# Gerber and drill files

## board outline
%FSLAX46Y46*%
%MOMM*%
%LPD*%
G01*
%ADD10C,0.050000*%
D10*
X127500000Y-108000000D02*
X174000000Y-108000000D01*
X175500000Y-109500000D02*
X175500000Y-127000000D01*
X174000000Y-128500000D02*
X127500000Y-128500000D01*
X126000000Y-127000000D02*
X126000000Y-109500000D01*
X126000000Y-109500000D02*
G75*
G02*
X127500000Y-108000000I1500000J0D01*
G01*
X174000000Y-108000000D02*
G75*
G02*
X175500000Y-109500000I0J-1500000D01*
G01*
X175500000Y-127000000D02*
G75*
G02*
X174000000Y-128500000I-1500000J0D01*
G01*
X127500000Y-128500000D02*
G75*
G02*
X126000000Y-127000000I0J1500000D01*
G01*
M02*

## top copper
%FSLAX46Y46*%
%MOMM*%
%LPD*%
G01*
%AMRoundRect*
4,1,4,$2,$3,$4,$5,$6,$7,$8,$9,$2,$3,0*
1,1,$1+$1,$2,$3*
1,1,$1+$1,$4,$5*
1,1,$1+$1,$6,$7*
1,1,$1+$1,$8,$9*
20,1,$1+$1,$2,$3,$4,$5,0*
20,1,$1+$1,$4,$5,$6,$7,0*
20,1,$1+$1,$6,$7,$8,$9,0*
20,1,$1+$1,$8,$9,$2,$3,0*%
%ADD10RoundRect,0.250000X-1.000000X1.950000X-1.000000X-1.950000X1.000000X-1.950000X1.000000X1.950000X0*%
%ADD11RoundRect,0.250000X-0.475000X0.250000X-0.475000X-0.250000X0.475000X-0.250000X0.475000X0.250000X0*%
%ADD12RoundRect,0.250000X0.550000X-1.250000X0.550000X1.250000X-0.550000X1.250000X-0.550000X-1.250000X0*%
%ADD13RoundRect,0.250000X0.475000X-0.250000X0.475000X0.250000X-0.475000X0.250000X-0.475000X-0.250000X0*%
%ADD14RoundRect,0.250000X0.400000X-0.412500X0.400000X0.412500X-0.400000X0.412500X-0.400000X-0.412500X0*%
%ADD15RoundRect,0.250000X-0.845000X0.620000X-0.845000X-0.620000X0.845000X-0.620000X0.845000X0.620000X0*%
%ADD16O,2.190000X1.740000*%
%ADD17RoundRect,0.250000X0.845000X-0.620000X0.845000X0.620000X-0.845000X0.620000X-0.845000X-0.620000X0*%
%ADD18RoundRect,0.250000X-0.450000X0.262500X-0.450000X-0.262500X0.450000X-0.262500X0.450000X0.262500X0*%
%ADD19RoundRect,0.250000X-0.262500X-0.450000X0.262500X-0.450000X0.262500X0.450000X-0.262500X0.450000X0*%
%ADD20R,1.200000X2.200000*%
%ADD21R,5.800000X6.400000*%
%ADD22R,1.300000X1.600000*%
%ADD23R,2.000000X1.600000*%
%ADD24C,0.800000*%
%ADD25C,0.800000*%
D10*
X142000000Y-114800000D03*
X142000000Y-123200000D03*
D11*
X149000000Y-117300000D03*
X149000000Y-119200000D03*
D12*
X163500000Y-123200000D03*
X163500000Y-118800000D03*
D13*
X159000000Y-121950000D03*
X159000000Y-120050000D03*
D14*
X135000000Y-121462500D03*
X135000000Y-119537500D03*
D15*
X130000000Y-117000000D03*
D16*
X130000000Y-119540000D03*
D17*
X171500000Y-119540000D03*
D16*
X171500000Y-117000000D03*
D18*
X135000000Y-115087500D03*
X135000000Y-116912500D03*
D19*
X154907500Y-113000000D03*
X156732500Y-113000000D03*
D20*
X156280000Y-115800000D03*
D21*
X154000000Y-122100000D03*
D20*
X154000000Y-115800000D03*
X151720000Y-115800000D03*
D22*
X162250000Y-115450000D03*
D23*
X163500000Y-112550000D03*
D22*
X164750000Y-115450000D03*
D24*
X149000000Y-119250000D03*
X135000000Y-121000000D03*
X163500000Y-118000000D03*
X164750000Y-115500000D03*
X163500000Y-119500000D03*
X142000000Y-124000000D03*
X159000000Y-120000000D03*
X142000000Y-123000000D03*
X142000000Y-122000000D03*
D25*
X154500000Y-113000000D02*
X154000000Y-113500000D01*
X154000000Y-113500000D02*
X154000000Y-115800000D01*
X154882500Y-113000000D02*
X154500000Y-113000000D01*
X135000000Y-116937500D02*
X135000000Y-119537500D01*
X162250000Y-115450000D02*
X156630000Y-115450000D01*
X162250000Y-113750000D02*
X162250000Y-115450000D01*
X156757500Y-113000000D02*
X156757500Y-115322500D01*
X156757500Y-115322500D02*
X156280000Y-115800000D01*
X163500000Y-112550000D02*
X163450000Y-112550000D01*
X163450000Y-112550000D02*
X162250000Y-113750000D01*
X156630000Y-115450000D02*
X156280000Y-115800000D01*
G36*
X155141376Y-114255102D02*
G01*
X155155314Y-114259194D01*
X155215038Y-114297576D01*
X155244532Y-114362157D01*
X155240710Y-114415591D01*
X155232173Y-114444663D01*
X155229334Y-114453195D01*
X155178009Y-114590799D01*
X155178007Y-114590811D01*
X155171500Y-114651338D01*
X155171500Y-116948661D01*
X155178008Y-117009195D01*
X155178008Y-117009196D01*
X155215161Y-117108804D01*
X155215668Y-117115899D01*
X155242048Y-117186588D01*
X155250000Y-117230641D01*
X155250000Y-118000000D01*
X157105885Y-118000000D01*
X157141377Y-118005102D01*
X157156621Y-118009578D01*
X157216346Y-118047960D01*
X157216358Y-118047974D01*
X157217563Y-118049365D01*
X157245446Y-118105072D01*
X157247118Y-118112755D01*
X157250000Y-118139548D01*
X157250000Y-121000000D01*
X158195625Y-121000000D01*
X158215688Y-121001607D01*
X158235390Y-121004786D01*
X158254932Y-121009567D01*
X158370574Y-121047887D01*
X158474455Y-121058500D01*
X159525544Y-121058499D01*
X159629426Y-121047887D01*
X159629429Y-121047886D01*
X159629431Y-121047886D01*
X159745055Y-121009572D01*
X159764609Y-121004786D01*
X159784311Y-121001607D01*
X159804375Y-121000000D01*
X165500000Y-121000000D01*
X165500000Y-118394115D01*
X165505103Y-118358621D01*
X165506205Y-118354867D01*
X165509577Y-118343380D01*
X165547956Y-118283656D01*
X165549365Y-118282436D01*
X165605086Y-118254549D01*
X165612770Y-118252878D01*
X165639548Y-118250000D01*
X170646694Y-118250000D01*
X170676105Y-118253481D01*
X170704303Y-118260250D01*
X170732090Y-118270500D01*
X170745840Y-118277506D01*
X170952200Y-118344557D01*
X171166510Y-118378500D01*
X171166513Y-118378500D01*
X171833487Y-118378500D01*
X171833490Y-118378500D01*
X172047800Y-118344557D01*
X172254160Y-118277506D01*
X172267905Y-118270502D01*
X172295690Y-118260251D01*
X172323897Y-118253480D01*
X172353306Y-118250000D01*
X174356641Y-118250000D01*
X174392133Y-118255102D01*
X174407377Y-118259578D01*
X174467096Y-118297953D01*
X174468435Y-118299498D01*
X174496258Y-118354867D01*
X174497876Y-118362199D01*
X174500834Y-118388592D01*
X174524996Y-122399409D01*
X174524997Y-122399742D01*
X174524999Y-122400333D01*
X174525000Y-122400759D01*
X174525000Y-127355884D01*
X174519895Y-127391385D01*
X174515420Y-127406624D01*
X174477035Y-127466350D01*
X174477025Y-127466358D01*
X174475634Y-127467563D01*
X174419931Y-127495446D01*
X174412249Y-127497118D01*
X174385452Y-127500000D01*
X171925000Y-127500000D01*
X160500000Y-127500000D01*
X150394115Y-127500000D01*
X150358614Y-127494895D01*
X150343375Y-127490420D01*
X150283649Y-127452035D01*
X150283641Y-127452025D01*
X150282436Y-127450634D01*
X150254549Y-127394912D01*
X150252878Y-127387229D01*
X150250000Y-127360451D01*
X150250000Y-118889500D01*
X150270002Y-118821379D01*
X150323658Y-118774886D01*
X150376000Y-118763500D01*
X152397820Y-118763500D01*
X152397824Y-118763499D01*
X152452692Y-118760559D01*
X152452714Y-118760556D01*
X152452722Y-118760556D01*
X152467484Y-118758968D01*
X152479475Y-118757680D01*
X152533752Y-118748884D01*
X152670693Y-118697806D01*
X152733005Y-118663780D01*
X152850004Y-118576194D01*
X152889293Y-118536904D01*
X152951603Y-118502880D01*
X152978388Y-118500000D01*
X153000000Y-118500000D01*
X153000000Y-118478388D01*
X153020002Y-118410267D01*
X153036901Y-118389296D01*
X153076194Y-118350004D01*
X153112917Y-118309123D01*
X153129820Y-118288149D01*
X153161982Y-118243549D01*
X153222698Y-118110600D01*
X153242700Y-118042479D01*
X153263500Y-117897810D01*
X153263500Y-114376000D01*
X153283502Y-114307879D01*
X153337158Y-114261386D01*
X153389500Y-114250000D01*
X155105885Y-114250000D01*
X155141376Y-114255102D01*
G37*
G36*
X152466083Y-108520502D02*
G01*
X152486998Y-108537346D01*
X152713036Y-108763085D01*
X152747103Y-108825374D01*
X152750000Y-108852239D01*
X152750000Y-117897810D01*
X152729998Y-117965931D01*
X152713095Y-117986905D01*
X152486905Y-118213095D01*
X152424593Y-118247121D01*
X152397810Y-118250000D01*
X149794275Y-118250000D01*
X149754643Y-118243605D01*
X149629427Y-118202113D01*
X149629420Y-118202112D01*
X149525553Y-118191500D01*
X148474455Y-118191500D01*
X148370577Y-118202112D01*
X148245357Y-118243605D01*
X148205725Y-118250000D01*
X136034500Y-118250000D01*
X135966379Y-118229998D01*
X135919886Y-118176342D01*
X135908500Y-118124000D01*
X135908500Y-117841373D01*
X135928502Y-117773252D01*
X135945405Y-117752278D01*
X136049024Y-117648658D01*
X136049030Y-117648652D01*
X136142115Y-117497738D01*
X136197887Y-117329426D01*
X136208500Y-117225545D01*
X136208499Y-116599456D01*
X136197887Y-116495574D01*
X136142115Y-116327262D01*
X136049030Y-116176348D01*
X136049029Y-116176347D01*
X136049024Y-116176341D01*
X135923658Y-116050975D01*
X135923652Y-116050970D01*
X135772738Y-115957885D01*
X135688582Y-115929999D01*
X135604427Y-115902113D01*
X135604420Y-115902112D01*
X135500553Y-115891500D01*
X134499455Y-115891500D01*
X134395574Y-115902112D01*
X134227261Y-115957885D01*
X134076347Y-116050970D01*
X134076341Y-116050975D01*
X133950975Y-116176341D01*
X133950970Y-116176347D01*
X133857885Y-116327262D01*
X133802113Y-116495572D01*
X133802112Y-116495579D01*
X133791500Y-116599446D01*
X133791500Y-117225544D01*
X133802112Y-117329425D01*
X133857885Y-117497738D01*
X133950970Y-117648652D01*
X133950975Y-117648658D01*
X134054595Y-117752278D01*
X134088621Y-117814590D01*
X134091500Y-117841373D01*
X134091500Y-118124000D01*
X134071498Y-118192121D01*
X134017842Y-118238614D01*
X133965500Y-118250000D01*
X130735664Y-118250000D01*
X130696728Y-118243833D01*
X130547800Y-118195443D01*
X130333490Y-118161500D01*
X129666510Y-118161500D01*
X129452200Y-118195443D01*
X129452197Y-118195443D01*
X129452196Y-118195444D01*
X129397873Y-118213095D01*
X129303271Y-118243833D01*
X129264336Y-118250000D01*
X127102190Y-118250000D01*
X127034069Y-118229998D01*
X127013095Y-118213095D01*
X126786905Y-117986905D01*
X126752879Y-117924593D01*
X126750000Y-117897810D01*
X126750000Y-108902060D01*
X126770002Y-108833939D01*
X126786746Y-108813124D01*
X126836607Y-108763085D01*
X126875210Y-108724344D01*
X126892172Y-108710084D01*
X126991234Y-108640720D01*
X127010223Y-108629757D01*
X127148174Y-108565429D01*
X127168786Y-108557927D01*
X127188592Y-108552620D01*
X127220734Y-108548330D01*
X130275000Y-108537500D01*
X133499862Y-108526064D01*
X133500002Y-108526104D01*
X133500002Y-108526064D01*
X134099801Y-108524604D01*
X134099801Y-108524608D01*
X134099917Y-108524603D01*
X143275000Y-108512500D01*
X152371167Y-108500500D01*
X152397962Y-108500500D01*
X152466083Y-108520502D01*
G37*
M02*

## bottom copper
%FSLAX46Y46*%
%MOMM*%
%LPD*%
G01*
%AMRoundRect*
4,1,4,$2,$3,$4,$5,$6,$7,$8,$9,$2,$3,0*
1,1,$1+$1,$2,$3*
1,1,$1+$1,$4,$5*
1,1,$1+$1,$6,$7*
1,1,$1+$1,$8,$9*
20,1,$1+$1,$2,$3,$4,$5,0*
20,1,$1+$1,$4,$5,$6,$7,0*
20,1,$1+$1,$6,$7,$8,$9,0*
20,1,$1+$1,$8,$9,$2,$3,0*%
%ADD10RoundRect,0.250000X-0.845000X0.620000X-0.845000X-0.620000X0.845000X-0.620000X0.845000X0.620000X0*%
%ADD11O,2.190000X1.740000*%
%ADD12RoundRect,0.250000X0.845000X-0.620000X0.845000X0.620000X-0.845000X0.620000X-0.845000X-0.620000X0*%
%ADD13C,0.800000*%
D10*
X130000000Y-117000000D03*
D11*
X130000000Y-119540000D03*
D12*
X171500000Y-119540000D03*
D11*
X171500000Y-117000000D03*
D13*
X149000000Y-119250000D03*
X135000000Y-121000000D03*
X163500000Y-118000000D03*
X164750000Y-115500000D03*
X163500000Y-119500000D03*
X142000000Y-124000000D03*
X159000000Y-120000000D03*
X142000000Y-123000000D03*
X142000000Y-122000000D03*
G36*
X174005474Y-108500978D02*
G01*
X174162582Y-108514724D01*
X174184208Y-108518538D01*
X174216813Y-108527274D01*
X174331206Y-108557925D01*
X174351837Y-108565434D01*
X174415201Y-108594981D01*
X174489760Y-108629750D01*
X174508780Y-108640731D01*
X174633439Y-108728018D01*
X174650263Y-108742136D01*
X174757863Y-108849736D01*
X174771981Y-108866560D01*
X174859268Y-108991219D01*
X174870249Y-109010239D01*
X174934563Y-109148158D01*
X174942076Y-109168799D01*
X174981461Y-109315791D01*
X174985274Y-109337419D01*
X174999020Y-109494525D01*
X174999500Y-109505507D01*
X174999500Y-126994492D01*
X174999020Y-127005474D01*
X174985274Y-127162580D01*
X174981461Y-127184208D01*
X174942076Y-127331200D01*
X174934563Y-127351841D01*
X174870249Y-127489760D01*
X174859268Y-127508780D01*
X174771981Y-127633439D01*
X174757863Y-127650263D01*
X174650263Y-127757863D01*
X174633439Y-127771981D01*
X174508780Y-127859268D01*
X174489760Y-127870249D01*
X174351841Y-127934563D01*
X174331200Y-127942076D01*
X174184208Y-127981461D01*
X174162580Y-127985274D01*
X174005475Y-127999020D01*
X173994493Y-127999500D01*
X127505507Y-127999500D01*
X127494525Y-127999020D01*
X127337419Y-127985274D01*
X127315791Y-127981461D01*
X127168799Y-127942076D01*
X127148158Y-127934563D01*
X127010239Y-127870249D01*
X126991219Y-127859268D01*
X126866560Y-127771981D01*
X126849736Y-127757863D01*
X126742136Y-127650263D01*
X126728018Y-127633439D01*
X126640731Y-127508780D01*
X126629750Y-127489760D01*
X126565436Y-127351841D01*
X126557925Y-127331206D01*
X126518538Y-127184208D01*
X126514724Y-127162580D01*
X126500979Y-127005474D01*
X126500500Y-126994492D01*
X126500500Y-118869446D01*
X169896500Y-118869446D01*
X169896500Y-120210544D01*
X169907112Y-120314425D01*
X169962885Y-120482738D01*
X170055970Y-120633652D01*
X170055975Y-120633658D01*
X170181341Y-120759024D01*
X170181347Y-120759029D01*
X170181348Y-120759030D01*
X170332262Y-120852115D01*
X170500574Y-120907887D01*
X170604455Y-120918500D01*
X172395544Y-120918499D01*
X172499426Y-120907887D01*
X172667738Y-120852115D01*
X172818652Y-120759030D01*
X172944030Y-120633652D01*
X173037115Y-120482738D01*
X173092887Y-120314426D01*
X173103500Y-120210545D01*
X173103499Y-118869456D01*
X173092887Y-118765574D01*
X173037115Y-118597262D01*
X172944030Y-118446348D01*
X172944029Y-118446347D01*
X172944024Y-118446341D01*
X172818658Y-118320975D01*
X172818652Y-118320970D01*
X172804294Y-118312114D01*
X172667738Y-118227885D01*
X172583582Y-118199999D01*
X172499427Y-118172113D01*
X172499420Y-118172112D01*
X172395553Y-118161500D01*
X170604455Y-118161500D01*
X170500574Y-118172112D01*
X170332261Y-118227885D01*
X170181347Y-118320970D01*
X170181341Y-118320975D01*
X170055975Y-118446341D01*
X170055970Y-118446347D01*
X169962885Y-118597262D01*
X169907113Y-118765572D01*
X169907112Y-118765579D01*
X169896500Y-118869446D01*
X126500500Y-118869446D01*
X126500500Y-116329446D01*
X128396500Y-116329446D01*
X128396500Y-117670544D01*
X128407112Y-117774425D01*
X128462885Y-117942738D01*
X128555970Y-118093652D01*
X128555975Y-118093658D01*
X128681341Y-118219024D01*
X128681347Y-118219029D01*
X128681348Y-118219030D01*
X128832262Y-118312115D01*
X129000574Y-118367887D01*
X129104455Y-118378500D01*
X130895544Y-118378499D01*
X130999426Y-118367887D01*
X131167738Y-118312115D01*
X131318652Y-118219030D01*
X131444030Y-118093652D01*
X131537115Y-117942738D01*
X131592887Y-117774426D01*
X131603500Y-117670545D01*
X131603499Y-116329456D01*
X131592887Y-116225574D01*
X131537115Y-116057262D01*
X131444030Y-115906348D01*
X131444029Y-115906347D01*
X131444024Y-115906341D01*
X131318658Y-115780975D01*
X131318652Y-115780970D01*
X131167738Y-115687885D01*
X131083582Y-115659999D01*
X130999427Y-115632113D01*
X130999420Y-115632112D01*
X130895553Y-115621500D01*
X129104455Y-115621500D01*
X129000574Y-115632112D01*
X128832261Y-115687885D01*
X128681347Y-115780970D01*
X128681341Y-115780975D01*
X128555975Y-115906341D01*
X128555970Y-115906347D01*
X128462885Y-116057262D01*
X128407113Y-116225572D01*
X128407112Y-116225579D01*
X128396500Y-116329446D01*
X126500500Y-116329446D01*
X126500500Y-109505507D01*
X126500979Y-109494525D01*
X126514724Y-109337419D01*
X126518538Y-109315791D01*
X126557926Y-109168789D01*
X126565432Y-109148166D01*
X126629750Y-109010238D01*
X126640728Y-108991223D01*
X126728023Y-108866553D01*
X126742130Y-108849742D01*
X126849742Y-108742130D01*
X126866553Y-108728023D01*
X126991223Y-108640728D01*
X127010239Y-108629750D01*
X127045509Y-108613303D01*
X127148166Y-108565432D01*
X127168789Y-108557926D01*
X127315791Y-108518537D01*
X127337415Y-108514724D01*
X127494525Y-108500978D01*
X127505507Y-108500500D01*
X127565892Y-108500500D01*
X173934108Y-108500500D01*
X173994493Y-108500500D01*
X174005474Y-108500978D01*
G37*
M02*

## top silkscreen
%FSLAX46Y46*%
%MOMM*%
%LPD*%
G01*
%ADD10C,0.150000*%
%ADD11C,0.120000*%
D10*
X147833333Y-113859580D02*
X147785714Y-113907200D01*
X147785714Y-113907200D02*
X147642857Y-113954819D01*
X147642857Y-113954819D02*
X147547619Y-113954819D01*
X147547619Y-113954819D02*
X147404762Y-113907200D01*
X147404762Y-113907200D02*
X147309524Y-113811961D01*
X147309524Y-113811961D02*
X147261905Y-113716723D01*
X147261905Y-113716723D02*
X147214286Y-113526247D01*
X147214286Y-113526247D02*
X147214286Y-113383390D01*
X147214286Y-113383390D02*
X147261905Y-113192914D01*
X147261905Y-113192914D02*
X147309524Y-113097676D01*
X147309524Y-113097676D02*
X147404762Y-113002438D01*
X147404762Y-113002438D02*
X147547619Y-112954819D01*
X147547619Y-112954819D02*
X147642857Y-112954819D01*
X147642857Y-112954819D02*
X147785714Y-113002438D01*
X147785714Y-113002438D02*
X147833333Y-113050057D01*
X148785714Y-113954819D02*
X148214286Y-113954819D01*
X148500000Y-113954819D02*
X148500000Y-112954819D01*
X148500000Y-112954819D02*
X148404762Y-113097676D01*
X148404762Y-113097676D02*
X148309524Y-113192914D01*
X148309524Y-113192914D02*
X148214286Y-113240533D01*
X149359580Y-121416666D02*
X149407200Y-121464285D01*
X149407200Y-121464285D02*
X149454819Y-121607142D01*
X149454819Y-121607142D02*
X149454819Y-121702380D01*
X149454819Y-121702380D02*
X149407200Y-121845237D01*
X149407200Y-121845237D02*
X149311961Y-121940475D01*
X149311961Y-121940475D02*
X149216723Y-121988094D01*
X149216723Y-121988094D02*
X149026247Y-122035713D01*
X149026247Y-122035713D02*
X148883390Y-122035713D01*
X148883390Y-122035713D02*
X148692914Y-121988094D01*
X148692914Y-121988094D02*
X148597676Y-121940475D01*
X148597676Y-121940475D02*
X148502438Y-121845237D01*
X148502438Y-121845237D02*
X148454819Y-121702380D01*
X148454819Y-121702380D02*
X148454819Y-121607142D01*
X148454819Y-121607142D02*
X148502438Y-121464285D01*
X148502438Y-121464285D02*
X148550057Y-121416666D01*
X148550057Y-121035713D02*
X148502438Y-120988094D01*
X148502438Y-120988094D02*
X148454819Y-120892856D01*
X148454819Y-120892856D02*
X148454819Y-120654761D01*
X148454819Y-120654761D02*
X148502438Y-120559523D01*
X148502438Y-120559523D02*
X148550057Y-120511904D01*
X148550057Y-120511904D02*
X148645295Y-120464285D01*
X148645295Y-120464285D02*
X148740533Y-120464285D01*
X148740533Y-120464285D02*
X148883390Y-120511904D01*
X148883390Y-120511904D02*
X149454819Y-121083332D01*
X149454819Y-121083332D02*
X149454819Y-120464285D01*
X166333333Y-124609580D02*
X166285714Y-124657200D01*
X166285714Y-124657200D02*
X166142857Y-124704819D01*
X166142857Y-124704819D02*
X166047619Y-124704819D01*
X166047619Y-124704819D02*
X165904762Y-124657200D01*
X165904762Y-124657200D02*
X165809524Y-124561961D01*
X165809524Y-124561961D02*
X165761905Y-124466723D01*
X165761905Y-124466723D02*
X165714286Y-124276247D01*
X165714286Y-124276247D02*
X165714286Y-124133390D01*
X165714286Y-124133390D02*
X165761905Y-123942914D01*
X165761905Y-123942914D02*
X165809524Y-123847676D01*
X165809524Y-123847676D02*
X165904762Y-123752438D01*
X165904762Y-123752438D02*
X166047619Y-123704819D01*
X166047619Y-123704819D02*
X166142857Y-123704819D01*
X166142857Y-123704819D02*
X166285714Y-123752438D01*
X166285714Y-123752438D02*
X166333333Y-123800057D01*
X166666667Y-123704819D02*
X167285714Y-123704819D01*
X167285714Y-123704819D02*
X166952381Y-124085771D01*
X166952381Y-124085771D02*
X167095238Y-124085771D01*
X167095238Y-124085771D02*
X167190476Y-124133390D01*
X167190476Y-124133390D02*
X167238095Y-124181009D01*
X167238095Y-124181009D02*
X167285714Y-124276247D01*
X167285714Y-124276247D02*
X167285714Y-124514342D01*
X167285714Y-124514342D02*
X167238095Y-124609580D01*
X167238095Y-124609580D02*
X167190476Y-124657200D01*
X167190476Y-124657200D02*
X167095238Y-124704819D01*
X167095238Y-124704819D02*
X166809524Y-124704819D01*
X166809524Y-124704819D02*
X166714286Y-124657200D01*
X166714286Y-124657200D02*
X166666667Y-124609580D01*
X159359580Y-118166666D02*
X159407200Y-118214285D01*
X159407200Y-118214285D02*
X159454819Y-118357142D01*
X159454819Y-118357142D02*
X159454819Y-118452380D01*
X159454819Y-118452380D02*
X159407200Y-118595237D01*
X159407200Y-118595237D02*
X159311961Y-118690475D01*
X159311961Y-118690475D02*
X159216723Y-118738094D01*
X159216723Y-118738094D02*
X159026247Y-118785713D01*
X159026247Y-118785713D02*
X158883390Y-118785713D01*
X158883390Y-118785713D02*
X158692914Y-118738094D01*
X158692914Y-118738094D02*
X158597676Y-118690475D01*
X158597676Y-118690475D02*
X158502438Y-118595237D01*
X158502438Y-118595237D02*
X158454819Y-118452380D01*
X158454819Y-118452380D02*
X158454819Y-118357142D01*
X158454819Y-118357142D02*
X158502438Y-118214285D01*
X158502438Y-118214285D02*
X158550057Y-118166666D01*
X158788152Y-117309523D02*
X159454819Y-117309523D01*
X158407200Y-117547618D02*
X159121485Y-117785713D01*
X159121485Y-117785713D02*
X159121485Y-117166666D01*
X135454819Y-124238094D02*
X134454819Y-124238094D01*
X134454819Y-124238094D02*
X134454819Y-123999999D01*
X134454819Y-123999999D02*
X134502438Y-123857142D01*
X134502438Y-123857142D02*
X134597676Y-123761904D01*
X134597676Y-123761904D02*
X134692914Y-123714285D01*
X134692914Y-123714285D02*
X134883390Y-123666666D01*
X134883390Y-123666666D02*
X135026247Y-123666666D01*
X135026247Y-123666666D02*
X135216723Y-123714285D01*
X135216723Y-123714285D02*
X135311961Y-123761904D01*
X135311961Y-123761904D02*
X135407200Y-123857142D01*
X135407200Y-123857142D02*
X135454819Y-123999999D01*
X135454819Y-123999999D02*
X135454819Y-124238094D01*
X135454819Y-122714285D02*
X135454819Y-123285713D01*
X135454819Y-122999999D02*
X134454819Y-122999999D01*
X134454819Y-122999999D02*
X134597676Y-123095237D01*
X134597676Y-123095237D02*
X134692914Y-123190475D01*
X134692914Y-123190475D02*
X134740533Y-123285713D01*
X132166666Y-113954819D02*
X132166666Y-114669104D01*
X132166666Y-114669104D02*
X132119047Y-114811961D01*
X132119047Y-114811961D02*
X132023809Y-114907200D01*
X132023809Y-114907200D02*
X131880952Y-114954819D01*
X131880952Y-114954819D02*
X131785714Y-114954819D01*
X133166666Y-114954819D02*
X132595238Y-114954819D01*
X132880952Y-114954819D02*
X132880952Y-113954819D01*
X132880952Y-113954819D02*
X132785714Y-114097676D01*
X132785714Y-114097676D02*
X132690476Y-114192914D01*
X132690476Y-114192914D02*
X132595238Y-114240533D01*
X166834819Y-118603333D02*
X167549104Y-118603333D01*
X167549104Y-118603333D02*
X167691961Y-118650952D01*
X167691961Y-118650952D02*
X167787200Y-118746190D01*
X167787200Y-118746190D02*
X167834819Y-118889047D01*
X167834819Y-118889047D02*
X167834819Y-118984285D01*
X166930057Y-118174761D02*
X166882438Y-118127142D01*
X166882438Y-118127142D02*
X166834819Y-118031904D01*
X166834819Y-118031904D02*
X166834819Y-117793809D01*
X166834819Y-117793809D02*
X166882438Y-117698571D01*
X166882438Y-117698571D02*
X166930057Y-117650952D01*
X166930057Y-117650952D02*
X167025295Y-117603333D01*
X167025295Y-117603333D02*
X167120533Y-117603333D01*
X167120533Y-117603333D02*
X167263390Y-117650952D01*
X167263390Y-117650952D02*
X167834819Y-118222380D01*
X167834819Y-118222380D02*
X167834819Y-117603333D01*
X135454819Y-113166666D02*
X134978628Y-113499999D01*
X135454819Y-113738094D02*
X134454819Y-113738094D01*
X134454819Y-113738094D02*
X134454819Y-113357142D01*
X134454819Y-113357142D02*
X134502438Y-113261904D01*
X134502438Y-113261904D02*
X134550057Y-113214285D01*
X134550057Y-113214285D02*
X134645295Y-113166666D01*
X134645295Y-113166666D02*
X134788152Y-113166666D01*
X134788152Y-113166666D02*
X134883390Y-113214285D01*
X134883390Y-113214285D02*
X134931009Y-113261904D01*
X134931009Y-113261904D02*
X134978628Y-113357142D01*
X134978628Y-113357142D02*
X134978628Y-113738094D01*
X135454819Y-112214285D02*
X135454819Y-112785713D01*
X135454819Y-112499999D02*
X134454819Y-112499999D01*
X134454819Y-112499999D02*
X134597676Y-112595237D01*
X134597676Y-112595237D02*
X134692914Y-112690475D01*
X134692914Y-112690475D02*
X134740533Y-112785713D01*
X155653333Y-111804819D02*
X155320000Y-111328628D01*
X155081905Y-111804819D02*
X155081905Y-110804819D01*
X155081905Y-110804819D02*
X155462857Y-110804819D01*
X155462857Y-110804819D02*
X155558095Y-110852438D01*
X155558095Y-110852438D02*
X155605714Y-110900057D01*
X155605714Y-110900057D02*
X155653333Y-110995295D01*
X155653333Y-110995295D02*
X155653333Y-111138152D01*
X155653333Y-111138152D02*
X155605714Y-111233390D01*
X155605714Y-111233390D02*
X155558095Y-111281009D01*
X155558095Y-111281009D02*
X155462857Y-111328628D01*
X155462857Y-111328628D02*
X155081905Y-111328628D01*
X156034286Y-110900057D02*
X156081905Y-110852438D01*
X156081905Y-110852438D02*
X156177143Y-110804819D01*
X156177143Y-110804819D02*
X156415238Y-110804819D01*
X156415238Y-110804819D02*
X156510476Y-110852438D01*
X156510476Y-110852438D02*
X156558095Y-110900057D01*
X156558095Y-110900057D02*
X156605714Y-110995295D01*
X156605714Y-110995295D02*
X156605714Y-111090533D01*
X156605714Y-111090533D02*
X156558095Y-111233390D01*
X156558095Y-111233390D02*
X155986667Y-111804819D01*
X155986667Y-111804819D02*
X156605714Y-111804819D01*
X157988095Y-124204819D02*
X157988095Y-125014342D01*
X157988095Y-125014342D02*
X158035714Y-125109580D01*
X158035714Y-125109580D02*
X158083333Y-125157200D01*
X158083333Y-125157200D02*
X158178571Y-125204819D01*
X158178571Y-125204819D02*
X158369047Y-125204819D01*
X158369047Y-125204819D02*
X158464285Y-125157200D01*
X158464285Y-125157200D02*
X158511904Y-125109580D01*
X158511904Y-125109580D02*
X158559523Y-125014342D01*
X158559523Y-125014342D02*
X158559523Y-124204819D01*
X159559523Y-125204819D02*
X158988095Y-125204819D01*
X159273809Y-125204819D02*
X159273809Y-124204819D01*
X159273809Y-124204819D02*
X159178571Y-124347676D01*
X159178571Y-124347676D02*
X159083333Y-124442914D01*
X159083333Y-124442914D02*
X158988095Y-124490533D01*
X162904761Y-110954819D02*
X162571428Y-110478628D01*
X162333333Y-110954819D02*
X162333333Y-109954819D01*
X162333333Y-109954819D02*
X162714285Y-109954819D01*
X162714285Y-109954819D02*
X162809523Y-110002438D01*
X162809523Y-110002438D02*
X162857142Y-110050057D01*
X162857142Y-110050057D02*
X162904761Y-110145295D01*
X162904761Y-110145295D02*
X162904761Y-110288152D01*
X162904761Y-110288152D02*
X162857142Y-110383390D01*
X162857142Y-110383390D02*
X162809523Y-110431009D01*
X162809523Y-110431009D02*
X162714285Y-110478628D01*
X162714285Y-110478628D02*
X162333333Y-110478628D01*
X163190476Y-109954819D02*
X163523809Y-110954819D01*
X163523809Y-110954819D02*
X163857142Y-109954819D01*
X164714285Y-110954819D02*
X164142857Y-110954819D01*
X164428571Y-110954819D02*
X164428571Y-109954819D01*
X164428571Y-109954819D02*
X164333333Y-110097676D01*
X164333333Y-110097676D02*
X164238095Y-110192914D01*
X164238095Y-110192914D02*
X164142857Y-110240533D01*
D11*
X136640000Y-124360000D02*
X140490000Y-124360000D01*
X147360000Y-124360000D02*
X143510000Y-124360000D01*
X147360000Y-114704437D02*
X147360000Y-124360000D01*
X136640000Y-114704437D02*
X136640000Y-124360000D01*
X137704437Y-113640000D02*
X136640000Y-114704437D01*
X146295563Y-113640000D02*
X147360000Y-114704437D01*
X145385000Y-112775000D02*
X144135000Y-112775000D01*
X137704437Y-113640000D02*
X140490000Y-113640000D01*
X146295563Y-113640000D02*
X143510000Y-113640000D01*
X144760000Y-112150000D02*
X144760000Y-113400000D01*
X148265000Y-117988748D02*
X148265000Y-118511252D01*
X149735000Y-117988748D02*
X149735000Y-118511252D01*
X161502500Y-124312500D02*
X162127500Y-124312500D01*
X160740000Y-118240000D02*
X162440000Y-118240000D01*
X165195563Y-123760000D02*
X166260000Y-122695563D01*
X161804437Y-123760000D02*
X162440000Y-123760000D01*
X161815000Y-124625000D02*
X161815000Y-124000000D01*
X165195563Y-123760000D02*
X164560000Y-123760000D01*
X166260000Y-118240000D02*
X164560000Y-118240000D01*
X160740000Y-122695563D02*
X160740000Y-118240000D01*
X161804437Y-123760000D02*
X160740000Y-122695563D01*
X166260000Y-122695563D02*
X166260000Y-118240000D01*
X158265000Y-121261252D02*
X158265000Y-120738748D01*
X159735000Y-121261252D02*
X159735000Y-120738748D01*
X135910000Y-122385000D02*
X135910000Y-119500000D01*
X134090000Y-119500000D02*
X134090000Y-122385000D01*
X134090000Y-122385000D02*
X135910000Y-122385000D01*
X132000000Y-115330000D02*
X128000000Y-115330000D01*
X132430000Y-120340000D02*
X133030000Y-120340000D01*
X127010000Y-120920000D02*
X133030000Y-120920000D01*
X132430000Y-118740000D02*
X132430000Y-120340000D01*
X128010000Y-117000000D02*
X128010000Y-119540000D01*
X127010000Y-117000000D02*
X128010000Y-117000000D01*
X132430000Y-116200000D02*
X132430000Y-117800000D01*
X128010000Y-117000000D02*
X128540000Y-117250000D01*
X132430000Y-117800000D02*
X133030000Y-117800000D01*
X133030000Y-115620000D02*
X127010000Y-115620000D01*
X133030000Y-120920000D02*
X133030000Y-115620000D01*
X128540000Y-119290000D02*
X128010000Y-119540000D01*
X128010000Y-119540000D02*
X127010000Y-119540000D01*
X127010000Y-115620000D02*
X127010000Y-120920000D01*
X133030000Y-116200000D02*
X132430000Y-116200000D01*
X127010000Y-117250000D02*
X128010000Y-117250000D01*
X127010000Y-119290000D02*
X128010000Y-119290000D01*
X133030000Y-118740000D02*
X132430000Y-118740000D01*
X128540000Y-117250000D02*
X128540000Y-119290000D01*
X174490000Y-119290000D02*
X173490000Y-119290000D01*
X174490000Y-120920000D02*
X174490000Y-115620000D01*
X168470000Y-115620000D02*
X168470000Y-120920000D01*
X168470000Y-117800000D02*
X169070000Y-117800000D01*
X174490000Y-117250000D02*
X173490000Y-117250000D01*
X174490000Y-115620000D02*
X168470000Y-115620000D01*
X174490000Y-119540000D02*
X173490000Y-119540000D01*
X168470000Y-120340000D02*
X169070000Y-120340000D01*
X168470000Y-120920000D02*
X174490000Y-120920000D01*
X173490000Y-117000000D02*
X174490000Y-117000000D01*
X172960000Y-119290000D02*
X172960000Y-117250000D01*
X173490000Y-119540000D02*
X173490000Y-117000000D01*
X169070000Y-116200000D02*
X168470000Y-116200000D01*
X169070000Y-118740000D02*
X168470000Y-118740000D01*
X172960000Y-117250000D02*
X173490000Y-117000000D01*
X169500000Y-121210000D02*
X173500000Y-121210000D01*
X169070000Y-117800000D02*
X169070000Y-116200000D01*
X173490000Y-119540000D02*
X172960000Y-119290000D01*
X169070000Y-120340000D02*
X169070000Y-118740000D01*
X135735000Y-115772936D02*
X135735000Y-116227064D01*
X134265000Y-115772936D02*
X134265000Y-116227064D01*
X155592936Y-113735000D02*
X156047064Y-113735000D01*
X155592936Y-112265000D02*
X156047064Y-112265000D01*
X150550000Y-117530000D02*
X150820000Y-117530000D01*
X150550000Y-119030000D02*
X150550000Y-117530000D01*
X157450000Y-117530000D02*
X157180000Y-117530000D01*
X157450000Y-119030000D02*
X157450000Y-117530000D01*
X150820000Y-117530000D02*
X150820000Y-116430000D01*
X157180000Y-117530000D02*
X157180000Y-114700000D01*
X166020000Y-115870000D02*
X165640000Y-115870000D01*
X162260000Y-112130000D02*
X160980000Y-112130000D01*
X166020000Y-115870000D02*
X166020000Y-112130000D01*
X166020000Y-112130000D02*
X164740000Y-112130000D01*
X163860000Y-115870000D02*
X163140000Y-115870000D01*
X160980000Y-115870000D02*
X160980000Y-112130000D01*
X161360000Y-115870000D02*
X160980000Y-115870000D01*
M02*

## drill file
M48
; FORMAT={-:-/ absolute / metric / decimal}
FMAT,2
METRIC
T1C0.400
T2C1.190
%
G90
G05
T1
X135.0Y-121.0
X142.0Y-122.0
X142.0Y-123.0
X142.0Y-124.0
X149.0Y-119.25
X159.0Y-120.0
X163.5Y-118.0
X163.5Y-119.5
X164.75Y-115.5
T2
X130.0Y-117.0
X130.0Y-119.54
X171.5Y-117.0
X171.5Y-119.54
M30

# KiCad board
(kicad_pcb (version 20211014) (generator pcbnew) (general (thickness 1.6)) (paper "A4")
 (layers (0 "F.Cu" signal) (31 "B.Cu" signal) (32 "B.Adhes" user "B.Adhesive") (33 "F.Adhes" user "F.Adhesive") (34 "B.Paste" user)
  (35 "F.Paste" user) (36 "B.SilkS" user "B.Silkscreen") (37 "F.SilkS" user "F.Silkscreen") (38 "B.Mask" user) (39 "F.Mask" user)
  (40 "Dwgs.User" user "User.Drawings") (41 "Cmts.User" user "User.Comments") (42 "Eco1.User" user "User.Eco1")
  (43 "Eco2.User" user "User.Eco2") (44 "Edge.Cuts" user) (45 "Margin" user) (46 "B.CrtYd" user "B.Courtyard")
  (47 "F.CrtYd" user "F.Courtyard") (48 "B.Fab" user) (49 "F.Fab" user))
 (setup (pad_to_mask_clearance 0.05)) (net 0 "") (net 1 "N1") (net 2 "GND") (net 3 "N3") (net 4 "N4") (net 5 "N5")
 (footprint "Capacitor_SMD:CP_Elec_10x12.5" (layer "F.Cu") (at 142 119 -90)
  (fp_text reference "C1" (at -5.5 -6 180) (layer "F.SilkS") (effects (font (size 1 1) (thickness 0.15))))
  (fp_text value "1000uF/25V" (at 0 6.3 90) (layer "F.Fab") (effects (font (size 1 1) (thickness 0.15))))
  (fp_line (start 5.36 5.36) (end 5.36 1.51) (layer "F.SilkS") (width 0.12))
  (fp_line (start 5.36 -5.36) (end 5.36 -1.51) (layer "F.SilkS") (width 0.12))
  (fp_line (start -4.295563 -5.36) (end 5.36 -5.36) (layer "F.SilkS") (width 0.12))
  (fp_line (start -4.295563 5.36) (end 5.36 5.36) (layer "F.SilkS") (width 0.12))
  (fp_line (start -5.36 4.295563) (end -4.295563 5.36) (layer "F.SilkS") (width 0.12))
  (fp_line (start -5.36 -4.295563) (end -4.295563 -5.36) (layer "F.SilkS") (width 0.12))
  (fp_line (start -6.225 -3.385) (end -6.225 -2.135) (layer "F.SilkS") (width 0.12))
  (fp_line (start -5.36 4.295563) (end -5.36 1.51) (layer "F.SilkS") (width 0.12))
  (fp_line (start -5.36 -4.295563) (end -5.36 -1.51) (layer "F.SilkS") (width 0.12))
  (fp_line (start -6.85 -2.76) (end -5.6 -2.76) (layer "F.SilkS") (width 0.12))
  (pad "1" smd roundrect (at -4.2 0 270) (size 4.4 2.5) (layers "F.Cu" "F.Paste" "F.Mask") (roundrect_rratio 0.1) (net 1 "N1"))
  (pad "2" smd roundrect (at 4.2 0 270) (size 4.4 2.5) (layers "F.Cu" "F.Paste" "F.Mask") (roundrect_rratio 0.1) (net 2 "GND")))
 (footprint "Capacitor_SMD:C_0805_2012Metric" (layer "F.Cu") (at 149 118.25 -90)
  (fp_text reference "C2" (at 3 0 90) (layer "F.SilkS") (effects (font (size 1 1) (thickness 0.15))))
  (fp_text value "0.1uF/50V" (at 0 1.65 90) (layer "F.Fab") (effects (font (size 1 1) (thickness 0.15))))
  (fp_line (start -0.261252 0.735) (end 0.261252 0.735) (layer "F.SilkS") (width 0.12))
  (fp_line (start -0.261252 -0.735) (end 0.261252 -0.735) (layer "F.SilkS") (width 0.12))
  (pad "1" smd roundrect (at -0.95 0 270) (size 1 1.45) (layers "F.Cu" "F.Paste" "F.Mask") (roundrect_rratio 0.25) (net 1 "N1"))
  (pad "2" smd roundrect (at 0.95 0 270) (size 1 1.45) (layers "F.Cu" "F.Paste" "F.Mask") (roundrect_rratio 0.25) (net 2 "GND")))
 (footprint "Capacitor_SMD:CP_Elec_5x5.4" (layer "F.Cu") (at 163.5 121 90)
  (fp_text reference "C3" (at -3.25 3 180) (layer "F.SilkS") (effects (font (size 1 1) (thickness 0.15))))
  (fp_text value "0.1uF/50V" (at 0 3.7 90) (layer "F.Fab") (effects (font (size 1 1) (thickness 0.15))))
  (fp_line (start -3.3125 -1.9975) (end -3.3125 -1.3725) (layer "F.SilkS") (width 0.12))
  (fp_line (start 2.76 -2.76) (end 2.76 -1.06) (layer "F.SilkS") (width 0.12))
  (fp_line (start -2.76 1.695563) (end -1.695563 2.76) (layer "F.SilkS") (width 0.12))
  (fp_line (start -2.76 -1.695563) (end -2.76 -1.06) (layer "F.SilkS") (width 0.12))
  (fp_line (start -3.625 -1.685) (end -3 -1.685) (layer "F.SilkS") (width 0.12))
  (fp_line (start -2.76 1.695563) (end -2.76 1.06) (layer "F.SilkS") (width 0.12))
  (fp_line (start 2.76 2.76) (end 2.76 1.06) (layer "F.SilkS") (width 0.12))
  (fp_line (start -1.695563 -2.76) (end 2.76 -2.76) (layer "F.SilkS") (width 0.12))
  (fp_line (start -2.76 -1.695563) (end -1.695563 -2.76) (layer "F.SilkS") (width 0.12))
  (fp_line (start -1.695563 2.76) (end 2.76 2.76) (layer "F.SilkS") (width 0.12))
  (pad "1" smd roundrect (at -2.2 0 90) (size 3 1.6) (layers "F.Cu" "F.Paste" "F.Mask") (roundrect_rratio 0.15625) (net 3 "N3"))
  (pad "2" smd roundrect (at 2.2 0 90) (size 3 1.6) (layers "F.Cu" "F.Paste" "F.Mask") (roundrect_rratio 0.15625) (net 2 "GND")))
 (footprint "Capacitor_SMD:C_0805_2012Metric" (layer "F.Cu") (at 159 121 90)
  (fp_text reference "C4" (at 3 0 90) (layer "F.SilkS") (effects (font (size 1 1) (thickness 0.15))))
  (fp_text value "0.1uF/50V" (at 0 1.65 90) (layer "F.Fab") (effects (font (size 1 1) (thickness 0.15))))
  (fp_line (start -0.261252 -0.735) (end 0.261252 -0.735) (layer "F.SilkS") (width 0.12))
  (fp_line (start -0.261252 0.735) (end 0.261252 0.735) (layer "F.SilkS") (width 0.12))
  (pad "1" smd roundrect (at -0.95 0 90) (size 1 1.45) (layers "F.Cu" "F.Paste" "F.Mask") (roundrect_rratio 0.25) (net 3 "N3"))
  (pad "2" smd roundrect (at 0.95 0 90) (size 1 1.45) (layers "F.Cu" "F.Paste" "F.Mask") (roundrect_rratio 0.25) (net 2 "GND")))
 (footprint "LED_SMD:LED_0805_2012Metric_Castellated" (layer "F.Cu") (at 135 120.5 90)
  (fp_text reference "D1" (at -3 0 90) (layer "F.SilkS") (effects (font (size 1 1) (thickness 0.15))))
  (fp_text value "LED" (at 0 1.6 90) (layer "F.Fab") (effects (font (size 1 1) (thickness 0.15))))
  (fp_line (start -1.885 0.91) (end 1 0.91) (layer "F.SilkS") (width 0.12))
  (fp_line (start 1 -0.91) (end -1.885 -0.91) (layer "F.SilkS") (width 0.12))
  (fp_line (start -1.885 -0.91) (end -1.885 0.91) (layer "F.SilkS") (width 0.12))
  (pad "1" smd roundrect locked (at -0.9625 0 90) (size 1.325 1.3) (layers "F.Cu" "F.Paste" "F.Mask") (roundrect_rratio 0.192308)
   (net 2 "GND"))
  (pad "2" smd roundrect locked (at 0.9625 0 90) (size 1.325 1.3) (layers "F.Cu" "F.Paste" "F.Mask") (roundrect_rratio 0.192308)
   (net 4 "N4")))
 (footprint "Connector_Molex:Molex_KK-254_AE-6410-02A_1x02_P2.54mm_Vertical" (layer "F.Cu") (at 130 117 -90)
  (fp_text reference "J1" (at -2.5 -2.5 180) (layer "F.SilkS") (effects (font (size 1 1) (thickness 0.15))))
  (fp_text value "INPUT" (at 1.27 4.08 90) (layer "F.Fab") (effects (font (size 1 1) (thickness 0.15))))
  (fp_line (start -1.67 -2) (end -1.67 2) (layer "F.SilkS") (width 0.12))
  (fp_line (start 3.34 -2.43) (end 3.34 -3.03) (layer "F.SilkS") (width 0.12))
  (fp_line (start 3.92 2.99) (end 3.92 -3.03) (layer "F.SilkS") (width 0.12))
  (fp_line (start 1.74 -2.43) (end 3.34 -2.43) (layer "F.SilkS") (width 0.12))
  (fp_line (start 0 1.99) (end 2.54 1.99) (layer "F.SilkS") (width 0.12))
  (fp_line (start 0 2.99) (end 0 1.99) (layer "F.SilkS") (width 0.12))
  (fp_line (start -0.8 -2.43) (end 0.8 -2.43) (layer "F.SilkS") (width 0.12))
  (fp_line (start 0 1.99) (end 0.25 1.46) (layer "F.SilkS") (width 0.12))
  (fp_line (start 0.8 -2.43) (end 0.8 -3.03) (layer "F.SilkS") (width 0.12))
  (fp_line (start -1.38 -3.03) (end -1.38 2.99) (layer "F.SilkS") (width 0.12))
  (fp_line (start 3.92 -3.03) (end -1.38 -3.03) (layer "F.SilkS") (width 0.12))
  (fp_line (start 2.29 1.46) (end 2.54 1.99) (layer "F.SilkS") (width 0.12))
  (fp_line (start 2.54 1.99) (end 2.54 2.99) (layer "F.SilkS") (width 0.12))
  (fp_line (start -1.38 2.99) (end 3.92 2.99) (layer "F.SilkS") (width 0.12))
  (fp_line (start -0.8 -3.03) (end -0.8 -2.43) (layer "F.SilkS") (width 0.12))
  (fp_line (start 0.25 2.99) (end 0.25 1.99) (layer "F.SilkS") (width 0.12))
  (fp_line (start 2.29 2.99) (end 2.29 1.99) (layer "F.SilkS") (width 0.12))
  (fp_line (start 1.74 -3.03) (end 1.74 -2.43) (layer "F.SilkS") (width 0.12))
  (fp_line (start 0.25 1.46) (end 2.29 1.46) (layer "F.SilkS") (width 0.12))
  (pad "1" thru_hole roundrect (at 0 0 270) (size 1.74 2.19) (drill 1.19) (layers *.Cu *.Mask) (roundrect_rratio 0.143678) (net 1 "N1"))
  (pad "2" thru_hole oval (at 2.54 0 270) (size 1.74 2.19) (drill 1.19) (layers *.Cu *.Mask) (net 2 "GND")))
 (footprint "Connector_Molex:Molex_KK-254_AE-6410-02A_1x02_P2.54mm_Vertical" (layer "F.Cu") (at 171.5 119.54 90)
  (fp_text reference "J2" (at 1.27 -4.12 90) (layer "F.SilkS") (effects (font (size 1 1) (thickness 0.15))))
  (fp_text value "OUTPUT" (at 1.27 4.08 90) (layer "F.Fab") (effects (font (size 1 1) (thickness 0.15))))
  (fp_line (start 0.25 2.99) (end 0.25 1.99) (layer "F.SilkS") (width 0.12))
  (fp_line (start -1.38 2.99) (end 3.92 2.99) (layer "F.SilkS") (width 0.12))
  (fp_line (start 3.92 -3.03) (end -1.38 -3.03) (layer "F.SilkS") (width 0.12))
  (fp_line (start 1.74 -3.03) (end 1.74 -2.43) (layer "F.SilkS") (width 0.12))
  (fp_line (start 2.29 2.99) (end 2.29 1.99) (layer "F.SilkS") (width 0.12))
  (fp_line (start 3.92 2.99) (end 3.92 -3.03) (layer "F.SilkS") (width 0.12))
  (fp_line (start 0 2.99) (end 0 1.99) (layer "F.SilkS") (width 0.12))
  (fp_line (start -0.8 -3.03) (end -0.8 -2.43) (layer "F.SilkS") (width 0.12))
  (fp_line (start -1.38 -3.03) (end -1.38 2.99) (layer "F.SilkS") (width 0.12))
  (fp_line (start 2.54 1.99) (end 2.54 2.99) (layer "F.SilkS") (width 0.12))
  (fp_line (start 0.25 1.46) (end 2.29 1.46) (layer "F.SilkS") (width 0.12))
  (fp_line (start 0 1.99) (end 2.54 1.99) (layer "F.SilkS") (width 0.12))
  (fp_line (start 3.34 -2.43) (end 3.34 -3.03) (layer "F.SilkS") (width 0.12))
  (fp_line (start 0.8 -2.43) (end 0.8 -3.03) (layer "F.SilkS") (width 0.12))
  (fp_line (start 2.29 1.46) (end 2.54 1.99) (layer "F.SilkS") (width 0.12))
  (fp_line (start -1.67 -2) (end -1.67 2) (layer "F.SilkS") (width 0.12))
  (fp_line (start 1.74 -2.43) (end 3.34 -2.43) (layer "F.SilkS") (width 0.12))
  (fp_line (start 0 1.99) (end 0.25 1.46) (layer "F.SilkS") (width 0.12))
  (fp_line (start -0.8 -2.43) (end 0.8 -2.43) (layer "F.SilkS") (width 0.12))
  (pad "1" thru_hole roundrect (at 0 0 90) (size 1.74 2.19) (drill 1.19) (layers *.Cu *.Mask) (roundrect_rratio 0.143678) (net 3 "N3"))
  (pad "2" thru_hole oval (at 2.54 0 90) (size 1.74 2.19) (drill 1.19) (layers *.Cu *.Mask) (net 2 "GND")))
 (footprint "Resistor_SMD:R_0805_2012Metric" (layer "F.Cu") (at 135 116 -90)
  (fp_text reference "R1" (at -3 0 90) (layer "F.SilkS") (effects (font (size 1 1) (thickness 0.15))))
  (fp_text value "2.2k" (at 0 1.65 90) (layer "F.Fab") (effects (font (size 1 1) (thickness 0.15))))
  (fp_line (start -0.227064 -0.735) (end 0.227064 -0.735) (layer "F.SilkS") (width 0.12))
  (fp_line (start -0.227064 0.735) (end 0.227064 0.735) (layer "F.SilkS") (width 0.12))
  (pad "1" smd roundrect (at -0.9125 0 270) (size 1.025 1.4) (layers "F.Cu" "F.Paste" "F.Mask") (roundrect_rratio 0.243902) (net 1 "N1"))
  (pad "2" smd roundrect (at 0.9125 0 270) (size 1.025 1.4) (layers "F.Cu" "F.Paste" "F.Mask") (roundrect_rratio 0.243902) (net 4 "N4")))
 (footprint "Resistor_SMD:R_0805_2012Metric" (layer "F.Cu") (at 155.82 113)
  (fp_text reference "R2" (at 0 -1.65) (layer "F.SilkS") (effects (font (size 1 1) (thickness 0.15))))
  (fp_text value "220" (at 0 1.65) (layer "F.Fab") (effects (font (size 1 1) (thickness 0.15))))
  (fp_line (start -0.227064 0.735) (end 0.227064 0.735) (layer "F.SilkS") (width 0.12))
  (fp_line (start -0.227064 -0.735) (end 0.227064 -0.735) (layer "F.SilkS") (width 0.12))
  (pad "1" smd roundrect (at -0.9125 0) (size 1.025 1.4) (layers "F.Cu" "F.Paste" "F.Mask") (roundrect_rratio 0.243902) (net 3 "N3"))
  (pad "2" smd roundrect (at 0.9125 0) (size 1.025 1.4) (layers "F.Cu" "F.Paste" "F.Mask") (roundrect_rratio 0.243902) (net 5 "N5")))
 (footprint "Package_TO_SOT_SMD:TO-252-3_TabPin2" (layer "F.Cu") (at 154 120 -90)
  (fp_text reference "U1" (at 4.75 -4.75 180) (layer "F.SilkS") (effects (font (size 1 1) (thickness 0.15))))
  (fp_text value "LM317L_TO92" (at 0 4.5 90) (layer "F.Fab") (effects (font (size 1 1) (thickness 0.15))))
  (fp_line (start -2.47 3.45) (end -2.47 3.18) (layer "F.SilkS") (width 0.12))
  (fp_line (start -0.97 3.45) (end -2.47 3.45) (layer "F.SilkS") (width 0.12))
  (fp_line (start -2.47 -3.45) (end -2.47 -3.18) (layer "F.SilkS") (width 0.12))
  (fp_line (start -0.97 -3.45) (end -2.47 -3.45) (layer "F.SilkS") (width 0.12))
  (fp_line (start -2.47 3.18) (end -3.57 3.18) (layer "F.SilkS") (width 0.12))
  (fp_line (start -2.47 -3.18) (end -5.3 -3.18) (layer "F.SilkS") (width 0.12))
  (pad "" smd rect (at 3.775 -1.525 270) (size 3.05 2.75) (layers "F.Paste"))
  (pad "" smd rect (at 0.425 -1.525 270) (size 3.05 2.75) (layers "F.Paste"))
  (pad "" smd rect (at 3.775 1.525 270) (size 3.05 2.75) (layers "F.Paste"))
  (pad "" smd rect (at 0.425 1.525 270) (size 3.05 2.75) (layers "F.Paste"))
  (pad "1" smd rect (at -4.2 -2.28 270) (size 2.2 1.2) (layers "F.Cu" "F.Paste" "F.Mask") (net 5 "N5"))
  (pad "2" smd rect (at 2.1 0 270) (size 6.4 5.8) (layers "F.Cu" "F.Mask") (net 3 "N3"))
  (pad "2" smd rect (at -4.2 0 270) (size 2.2 1.2) (layers "F.Cu" "F.Paste" "F.Mask") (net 3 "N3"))
  (pad "3" smd rect (at -4.2 2.28 270) (size 2.2 1.2) (layers "F.Cu" "F.Paste" "F.Mask") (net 1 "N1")))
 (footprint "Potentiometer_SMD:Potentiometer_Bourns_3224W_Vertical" (layer "F.Cu") (at 163.5 114 180)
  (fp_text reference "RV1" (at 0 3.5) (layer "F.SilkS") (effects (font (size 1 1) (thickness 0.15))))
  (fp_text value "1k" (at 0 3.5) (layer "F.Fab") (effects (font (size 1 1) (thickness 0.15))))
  (fp_line (start -2.52 -1.87) (end -2.14 -1.87) (layer "F.SilkS") (width 0.12))
  (fp_line (start 1.24 1.87) (end 2.52 1.87) (layer "F.SilkS") (width 0.12))
  (fp_line (start -2.52 -1.87) (end -2.52 1.87) (layer "F.SilkS") (width 0.12))
  (fp_line (start -2.52 1.87) (end -1.24 1.87) (layer "F.SilkS") (width 0.12))
  (fp_line (start -0.36 -1.87) (end 0.36 -1.87) (layer "F.SilkS") (width 0.12))
  (fp_line (start 2.52 -1.87) (end 2.52 1.87) (layer "F.SilkS") (width 0.12))
  (fp_line (start 2.14 -1.87) (end 2.52 -1.87) (layer "F.SilkS") (width 0.12))
  (pad "1" smd rect (at 1.25 -1.45 180) (size 1.3 1.6) (layers "F.Cu" "F.Paste" "F.Mask") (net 5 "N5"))
  (pad "2" smd rect (at 0 1.45 180) (size 2 1.6) (layers "F.Cu" "F.Paste" "F.Mask") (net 5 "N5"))
  (pad "3" smd rect (at -1.25 -1.45 180) (size 1.3 1.6) (layers "F.Cu" "F.Paste" "F.Mask") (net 2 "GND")))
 (gr_line (start 127.5 108) (end 174 108) (layer "Edge.Cuts") (width 0.05))
 (gr_line (start 175.5 109.5) (end 175.5 127) (layer "Edge.Cuts") (width 0.05))
 (gr_line (start 174 128.5) (end 127.5 128.5) (layer "Edge.Cuts") (width 0.05))
 (gr_line (start 126 127) (end 126 109.5) (layer "Edge.Cuts") (width 0.05))
 (gr_arc (start 126 109.5) (mid 126.43934 108.43934) (end 127.5 108) (layer "Edge.Cuts") (width 0.05))
 (gr_arc (start 174 108) (mid 175.06066 108.43934) (end 175.5 109.5) (layer "Edge.Cuts") (width 0.05))
 (gr_arc (start 175.5 127) (mid 175.06066 128.06066) (end 174 128.5) (layer "Edge.Cuts") (width 0.05))
 (gr_arc (start 127.5 128.5) (mid 126.43934 128.06066) (end 126 127) (layer "Edge.Cuts") (width 0.05))
 (via (at 149 119.25) (size 0.8) (drill 0.4) (layers "F.Cu" "B.Cu") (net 2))
 (via (at 135 121) (size 0.8) (drill 0.4) (layers "F.Cu" "B.Cu") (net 2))
 (via (at 163.5 118) (size 0.8) (drill 0.4) (layers "F.Cu" "B.Cu") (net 2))
 (via (at 164.75 115.5) (size 0.8) (drill 0.4) (layers "F.Cu" "B.Cu") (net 2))
 (via (at 163.5 119.5) (size 0.8) (drill 0.4) (layers "F.Cu" "B.Cu") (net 2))
 (via (at 142 124) (size 0.8) (drill 0.4) (layers "F.Cu" "B.Cu") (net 2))
 (via (at 159 120) (size 0.8) (drill 0.4) (layers "F.Cu" "B.Cu") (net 2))
 (via (at 142 123) (size 0.8) (drill 0.4) (layers "F.Cu" "B.Cu") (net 2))
 (via (at 142 122) (size 0.8) (drill 0.4) (layers "F.Cu" "B.Cu") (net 2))
 (segment (start 154.5 113) (end 154 113.5) (width 0.8) (layer "F.Cu") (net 3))
 (segment (start 154 113.5) (end 154 115.8) (width 0.8) (layer "F.Cu") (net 3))
 (segment (start 154.8825 113) (end 154.5 113) (width 0.8) (layer "F.Cu") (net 3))
 (segment (start 135 116.9375) (end 135 119.5375) (width 0.8) (layer "F.Cu") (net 4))
 (segment (start 162.25 115.45) (end 156.63 115.45) (width 0.8) (layer "F.Cu") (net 5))
 (segment (start 162.25 113.75) (end 162.25 115.45) (width 0.8) (layer "F.Cu") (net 5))
 (segment (start 156.7575 113) (end 156.7575 115.3225) (width 0.8) (layer "F.Cu") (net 5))
 (segment (start 156.7575 115.3225) (end 156.28 115.8) (width 0.8) (layer "F.Cu") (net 5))
 (segment (start 163.5 112.55) (end 163.45 112.55) (width 0.8) (layer "F.Cu") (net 5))
 (segment (start 163.45 112.55) (end 162.25 113.75) (width 0.8) (layer "F.Cu") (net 5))
 (segment (start 156.63 115.45) (end 156.28 115.8) (width 0.8) (layer "F.Cu") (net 5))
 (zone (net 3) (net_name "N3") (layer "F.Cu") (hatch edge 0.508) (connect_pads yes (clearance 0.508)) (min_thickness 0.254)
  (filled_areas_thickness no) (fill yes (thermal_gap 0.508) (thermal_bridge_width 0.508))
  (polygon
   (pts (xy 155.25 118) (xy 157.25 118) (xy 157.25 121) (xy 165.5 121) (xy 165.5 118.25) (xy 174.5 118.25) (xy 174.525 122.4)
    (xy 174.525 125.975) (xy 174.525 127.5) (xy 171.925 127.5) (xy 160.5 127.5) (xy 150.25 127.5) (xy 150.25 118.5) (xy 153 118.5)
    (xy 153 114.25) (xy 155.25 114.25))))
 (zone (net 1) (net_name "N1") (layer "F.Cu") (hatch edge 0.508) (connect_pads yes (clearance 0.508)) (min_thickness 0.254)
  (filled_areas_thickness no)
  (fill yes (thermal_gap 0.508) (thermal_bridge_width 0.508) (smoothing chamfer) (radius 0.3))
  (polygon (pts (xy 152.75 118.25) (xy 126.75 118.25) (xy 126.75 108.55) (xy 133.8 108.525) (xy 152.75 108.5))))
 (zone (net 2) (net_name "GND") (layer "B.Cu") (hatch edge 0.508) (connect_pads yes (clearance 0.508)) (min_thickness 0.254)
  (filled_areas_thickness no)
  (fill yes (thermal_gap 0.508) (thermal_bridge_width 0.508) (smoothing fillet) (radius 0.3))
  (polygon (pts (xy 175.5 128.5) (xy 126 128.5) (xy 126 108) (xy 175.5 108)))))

